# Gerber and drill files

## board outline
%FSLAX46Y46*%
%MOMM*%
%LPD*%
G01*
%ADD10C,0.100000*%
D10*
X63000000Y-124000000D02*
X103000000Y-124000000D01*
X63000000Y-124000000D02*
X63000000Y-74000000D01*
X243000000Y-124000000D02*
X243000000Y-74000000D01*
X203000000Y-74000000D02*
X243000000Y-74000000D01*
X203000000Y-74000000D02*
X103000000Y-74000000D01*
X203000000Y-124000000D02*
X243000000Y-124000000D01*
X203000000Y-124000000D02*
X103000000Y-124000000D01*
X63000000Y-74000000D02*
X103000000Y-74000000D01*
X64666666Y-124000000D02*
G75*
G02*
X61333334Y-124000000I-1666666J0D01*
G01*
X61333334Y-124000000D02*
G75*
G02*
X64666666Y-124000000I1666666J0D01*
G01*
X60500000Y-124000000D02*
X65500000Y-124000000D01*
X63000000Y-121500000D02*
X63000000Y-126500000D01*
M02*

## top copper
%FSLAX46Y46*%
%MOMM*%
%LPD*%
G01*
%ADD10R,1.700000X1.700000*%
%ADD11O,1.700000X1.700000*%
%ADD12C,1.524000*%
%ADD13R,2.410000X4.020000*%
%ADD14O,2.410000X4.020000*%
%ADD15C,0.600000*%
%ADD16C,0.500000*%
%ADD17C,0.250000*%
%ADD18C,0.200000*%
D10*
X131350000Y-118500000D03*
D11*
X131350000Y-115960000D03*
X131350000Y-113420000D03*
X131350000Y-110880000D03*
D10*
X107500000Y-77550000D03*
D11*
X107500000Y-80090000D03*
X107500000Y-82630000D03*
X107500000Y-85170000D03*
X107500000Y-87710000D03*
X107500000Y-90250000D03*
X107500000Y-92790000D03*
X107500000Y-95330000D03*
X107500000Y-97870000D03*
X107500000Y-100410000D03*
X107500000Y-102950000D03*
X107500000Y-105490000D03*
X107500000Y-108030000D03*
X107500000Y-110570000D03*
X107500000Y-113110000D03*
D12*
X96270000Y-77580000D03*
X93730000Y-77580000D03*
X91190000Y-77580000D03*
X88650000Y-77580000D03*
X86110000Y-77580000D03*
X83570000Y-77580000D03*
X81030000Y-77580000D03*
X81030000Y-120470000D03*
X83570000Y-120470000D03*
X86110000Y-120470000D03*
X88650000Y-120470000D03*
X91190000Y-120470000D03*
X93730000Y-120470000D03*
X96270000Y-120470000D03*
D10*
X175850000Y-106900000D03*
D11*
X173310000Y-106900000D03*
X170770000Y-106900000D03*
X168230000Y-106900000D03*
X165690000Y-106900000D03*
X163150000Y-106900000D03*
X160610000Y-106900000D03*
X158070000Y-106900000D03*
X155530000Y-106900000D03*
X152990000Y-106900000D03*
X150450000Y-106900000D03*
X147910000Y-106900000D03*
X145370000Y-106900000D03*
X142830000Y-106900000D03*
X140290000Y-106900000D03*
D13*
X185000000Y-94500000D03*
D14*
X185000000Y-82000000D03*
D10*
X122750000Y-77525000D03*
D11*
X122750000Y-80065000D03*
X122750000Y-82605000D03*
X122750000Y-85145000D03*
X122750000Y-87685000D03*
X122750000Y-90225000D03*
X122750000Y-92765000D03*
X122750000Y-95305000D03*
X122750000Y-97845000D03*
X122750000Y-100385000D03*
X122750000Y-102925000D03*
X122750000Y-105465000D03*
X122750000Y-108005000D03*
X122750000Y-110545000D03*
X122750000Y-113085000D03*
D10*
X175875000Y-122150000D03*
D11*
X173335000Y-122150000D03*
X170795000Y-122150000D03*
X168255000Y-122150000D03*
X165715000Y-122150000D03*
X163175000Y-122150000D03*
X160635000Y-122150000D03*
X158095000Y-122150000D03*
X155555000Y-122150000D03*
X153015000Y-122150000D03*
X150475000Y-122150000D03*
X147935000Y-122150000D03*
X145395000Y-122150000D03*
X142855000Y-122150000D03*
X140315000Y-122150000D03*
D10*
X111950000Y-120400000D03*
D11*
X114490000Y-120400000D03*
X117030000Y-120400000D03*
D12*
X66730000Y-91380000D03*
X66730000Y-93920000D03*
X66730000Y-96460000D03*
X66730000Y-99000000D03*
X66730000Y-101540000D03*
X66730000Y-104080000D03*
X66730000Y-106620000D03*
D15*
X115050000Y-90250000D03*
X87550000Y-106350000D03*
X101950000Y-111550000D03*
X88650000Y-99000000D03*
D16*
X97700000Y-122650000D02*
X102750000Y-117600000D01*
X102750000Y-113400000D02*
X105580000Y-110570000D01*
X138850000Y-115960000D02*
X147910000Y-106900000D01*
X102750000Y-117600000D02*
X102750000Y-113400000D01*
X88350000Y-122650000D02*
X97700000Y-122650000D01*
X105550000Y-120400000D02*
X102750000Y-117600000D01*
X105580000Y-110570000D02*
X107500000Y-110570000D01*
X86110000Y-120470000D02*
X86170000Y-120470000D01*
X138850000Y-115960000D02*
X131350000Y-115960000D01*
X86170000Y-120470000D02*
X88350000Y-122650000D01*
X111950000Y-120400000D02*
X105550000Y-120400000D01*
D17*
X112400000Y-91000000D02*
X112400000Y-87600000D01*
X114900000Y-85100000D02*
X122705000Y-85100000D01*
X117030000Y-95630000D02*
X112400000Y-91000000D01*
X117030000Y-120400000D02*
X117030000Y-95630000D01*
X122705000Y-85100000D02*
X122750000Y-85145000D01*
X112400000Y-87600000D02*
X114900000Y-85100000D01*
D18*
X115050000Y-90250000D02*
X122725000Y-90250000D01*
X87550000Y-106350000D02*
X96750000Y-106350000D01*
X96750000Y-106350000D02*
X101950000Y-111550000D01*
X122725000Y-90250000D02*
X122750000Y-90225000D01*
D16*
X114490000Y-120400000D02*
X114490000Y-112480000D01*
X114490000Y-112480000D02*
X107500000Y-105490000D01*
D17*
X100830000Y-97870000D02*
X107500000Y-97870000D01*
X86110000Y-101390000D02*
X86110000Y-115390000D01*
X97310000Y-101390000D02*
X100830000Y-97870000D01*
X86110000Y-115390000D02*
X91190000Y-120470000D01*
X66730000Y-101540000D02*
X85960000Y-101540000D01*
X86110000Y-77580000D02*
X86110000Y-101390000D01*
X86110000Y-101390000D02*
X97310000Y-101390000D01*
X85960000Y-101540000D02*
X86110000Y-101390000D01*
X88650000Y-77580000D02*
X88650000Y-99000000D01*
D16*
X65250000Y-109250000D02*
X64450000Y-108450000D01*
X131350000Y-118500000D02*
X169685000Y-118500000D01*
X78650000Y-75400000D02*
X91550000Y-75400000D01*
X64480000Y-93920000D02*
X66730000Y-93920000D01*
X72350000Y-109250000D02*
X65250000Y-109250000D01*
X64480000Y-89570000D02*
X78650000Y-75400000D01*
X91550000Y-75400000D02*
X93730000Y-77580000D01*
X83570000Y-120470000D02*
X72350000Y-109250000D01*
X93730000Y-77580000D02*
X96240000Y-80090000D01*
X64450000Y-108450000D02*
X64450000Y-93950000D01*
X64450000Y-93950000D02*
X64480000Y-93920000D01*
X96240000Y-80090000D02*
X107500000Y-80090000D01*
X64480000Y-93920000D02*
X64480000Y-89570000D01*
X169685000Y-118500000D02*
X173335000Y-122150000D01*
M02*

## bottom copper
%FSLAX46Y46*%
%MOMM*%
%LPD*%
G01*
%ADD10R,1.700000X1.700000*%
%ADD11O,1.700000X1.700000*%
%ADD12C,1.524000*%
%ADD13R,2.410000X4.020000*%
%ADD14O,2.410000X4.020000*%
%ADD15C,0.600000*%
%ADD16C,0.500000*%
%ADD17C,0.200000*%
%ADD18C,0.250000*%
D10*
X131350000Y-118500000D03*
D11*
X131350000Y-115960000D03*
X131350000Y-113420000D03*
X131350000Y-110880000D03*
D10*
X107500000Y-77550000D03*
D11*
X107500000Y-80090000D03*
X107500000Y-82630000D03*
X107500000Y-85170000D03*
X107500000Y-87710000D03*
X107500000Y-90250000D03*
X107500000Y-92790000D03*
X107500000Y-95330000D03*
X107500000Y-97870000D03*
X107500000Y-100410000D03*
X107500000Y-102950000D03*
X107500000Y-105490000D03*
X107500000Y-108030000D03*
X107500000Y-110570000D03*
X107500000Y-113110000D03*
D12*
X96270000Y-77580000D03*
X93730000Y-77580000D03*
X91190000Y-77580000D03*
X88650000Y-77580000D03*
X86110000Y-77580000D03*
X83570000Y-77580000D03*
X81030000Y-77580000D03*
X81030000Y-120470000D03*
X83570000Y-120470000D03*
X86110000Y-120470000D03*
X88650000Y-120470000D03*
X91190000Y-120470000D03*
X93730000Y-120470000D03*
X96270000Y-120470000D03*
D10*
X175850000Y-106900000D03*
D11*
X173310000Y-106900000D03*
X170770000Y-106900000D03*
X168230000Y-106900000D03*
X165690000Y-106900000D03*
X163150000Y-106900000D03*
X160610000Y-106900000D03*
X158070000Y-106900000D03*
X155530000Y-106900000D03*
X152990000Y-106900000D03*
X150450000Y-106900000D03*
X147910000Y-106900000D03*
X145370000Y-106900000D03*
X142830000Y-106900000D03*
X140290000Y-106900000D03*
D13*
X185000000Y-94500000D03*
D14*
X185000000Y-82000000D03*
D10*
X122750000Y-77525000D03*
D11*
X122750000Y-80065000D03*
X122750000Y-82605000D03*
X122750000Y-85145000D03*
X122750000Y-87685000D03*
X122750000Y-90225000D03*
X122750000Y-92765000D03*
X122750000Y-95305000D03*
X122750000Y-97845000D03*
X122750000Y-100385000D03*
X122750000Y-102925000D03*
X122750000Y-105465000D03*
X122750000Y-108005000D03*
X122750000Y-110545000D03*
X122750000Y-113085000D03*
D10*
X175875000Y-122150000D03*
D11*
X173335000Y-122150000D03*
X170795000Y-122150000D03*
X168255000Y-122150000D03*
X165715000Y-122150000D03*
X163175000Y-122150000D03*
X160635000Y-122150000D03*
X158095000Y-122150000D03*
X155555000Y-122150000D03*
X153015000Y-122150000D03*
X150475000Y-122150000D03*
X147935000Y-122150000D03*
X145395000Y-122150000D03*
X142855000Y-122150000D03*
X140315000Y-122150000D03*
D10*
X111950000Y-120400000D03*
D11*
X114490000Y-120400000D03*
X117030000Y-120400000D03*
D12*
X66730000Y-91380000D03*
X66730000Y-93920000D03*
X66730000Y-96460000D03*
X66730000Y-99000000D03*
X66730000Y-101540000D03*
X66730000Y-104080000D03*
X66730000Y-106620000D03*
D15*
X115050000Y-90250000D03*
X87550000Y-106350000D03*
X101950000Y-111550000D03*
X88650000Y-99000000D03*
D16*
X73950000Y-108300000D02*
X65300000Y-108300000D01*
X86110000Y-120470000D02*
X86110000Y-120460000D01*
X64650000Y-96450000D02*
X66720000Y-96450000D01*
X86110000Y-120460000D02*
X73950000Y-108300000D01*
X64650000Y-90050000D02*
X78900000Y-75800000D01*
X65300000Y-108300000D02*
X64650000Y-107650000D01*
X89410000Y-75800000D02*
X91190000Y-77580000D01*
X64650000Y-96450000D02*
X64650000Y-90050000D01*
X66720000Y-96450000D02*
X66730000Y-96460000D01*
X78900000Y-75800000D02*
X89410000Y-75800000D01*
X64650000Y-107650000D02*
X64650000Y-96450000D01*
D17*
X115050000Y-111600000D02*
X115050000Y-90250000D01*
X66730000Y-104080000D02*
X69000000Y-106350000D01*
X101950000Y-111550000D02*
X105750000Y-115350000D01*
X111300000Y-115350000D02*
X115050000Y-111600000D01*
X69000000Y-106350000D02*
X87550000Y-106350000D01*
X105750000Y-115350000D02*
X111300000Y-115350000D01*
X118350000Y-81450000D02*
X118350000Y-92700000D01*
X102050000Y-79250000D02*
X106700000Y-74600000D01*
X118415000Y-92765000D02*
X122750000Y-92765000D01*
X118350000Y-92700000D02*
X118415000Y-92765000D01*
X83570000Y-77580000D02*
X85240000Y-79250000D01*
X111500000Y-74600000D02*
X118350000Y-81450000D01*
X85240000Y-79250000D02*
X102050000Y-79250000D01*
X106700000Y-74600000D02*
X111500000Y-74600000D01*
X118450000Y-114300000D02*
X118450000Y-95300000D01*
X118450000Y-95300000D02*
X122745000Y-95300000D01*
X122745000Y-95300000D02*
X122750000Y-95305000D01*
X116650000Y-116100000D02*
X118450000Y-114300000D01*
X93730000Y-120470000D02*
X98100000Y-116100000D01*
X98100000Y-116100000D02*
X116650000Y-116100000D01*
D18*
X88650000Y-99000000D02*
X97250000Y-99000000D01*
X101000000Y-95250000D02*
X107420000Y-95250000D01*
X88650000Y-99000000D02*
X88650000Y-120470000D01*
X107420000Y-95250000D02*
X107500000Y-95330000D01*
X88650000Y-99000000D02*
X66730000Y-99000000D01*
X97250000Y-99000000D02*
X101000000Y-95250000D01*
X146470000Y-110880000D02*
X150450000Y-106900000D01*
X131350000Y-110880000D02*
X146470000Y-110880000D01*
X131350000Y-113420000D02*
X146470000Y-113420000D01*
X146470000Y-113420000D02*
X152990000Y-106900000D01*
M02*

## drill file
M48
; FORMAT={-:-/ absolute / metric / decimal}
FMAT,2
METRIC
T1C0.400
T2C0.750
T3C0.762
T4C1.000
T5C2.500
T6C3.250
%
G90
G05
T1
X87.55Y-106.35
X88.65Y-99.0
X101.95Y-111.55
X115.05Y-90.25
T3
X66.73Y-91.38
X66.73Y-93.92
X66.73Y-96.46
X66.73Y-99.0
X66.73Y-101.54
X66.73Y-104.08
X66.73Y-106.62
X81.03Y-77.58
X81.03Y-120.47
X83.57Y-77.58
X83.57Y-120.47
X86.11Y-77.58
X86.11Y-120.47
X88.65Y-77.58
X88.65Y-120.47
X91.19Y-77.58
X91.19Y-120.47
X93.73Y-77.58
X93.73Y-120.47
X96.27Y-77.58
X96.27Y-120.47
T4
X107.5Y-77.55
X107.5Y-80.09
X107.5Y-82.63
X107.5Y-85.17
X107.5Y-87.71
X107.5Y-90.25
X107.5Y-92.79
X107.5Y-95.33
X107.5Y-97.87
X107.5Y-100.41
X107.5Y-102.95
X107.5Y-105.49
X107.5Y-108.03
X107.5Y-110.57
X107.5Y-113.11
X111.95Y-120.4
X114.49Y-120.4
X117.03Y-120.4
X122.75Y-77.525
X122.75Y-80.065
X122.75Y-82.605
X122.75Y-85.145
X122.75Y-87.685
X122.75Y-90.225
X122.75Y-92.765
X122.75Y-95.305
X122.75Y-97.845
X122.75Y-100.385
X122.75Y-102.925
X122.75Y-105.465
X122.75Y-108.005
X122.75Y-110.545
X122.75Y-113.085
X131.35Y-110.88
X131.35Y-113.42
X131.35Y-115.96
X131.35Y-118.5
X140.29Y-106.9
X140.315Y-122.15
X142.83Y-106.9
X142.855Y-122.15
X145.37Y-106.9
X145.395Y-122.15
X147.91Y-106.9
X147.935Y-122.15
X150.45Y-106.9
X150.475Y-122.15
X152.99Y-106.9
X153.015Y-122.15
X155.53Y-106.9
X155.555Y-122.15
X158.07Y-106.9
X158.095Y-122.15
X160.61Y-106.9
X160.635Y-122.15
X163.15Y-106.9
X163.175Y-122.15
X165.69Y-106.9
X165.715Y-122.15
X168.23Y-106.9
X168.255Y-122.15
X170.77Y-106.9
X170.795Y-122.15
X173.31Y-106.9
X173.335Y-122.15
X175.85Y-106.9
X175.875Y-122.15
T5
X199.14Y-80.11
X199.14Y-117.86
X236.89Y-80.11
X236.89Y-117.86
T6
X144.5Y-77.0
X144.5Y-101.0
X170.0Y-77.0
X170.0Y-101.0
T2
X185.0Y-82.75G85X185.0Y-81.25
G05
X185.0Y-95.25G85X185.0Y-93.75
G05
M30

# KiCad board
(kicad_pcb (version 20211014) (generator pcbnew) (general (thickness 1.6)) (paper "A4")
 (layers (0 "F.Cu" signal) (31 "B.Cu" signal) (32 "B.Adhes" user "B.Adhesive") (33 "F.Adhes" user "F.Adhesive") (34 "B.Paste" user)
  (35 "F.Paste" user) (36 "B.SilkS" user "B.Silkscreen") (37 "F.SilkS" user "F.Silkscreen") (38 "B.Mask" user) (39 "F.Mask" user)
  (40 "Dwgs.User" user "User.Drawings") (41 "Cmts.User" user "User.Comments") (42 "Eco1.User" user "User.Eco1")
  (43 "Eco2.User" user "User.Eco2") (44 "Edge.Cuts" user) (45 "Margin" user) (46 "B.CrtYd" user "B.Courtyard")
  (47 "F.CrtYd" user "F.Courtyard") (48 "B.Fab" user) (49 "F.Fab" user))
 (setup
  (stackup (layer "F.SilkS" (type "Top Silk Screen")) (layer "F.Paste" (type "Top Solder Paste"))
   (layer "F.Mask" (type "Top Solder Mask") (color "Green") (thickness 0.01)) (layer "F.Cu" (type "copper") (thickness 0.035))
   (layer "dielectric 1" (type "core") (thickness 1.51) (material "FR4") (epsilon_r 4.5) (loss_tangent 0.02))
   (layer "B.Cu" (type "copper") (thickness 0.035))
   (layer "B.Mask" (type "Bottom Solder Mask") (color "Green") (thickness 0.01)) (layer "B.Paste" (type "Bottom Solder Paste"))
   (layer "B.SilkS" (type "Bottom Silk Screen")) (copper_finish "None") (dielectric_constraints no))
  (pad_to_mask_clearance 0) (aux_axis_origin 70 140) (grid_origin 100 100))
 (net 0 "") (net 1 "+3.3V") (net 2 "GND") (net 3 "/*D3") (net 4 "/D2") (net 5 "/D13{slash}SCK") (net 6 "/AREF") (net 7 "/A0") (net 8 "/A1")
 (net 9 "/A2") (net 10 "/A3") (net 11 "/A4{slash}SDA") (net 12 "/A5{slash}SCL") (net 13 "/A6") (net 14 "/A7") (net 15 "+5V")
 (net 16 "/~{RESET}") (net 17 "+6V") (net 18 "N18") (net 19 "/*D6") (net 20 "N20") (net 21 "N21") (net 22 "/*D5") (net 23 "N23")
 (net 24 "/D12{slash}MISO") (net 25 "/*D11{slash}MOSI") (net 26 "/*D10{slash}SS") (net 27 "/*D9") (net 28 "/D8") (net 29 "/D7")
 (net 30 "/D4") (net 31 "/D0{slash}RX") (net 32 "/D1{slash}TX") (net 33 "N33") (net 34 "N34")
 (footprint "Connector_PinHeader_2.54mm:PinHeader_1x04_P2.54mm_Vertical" (layer "F.Cu") (at 131.35 118.5 180)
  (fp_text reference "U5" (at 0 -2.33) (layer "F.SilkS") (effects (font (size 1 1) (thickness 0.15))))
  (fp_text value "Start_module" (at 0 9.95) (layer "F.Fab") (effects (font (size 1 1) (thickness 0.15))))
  (pad "1" thru_hole rect (at 0 0 180) (size 1.7 1.7) (drill 1) (layers *.Cu *.Mask) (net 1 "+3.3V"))
  (pad "2" thru_hole oval (at 0 2.54 180) (size 1.7 1.7) (drill 1) (layers *.Cu *.Mask) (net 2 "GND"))
  (pad "3" thru_hole oval (at 0 5.08 180) (size 1.7 1.7) (drill 1) (layers *.Cu *.Mask) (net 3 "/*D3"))
  (pad "4" thru_hole oval (at 0 7.62 180) (size 1.7 1.7) (drill 1) (layers *.Cu *.Mask) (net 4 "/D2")))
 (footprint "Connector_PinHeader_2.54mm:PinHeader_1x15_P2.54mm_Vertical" (layer "F.Cu") (at 107.5 77.55)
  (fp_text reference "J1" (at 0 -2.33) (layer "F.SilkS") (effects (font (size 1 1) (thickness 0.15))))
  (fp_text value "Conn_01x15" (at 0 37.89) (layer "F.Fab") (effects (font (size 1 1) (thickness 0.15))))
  (pad "1" thru_hole rect (at 0 0) (size 1.7 1.7) (drill 1) (layers *.Cu *.Mask) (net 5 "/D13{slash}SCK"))
  (pad "2" thru_hole oval (at 0 2.54) (size 1.7 1.7) (drill 1) (layers *.Cu *.Mask) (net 1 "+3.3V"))
  (pad "3" thru_hole oval (at 0 5.08) (size 1.7 1.7) (drill 1) (layers *.Cu *.Mask) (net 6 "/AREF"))
  (pad "4" thru_hole oval (at 0 7.62) (size 1.7 1.7) (drill 1) (layers *.Cu *.Mask) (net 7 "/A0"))
  (pad "5" thru_hole oval (at 0 10.16) (size 1.7 1.7) (drill 1) (layers *.Cu *.Mask) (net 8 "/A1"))
  (pad "6" thru_hole oval (at 0 12.7) (size 1.7 1.7) (drill 1) (layers *.Cu *.Mask) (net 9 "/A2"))
  (pad "7" thru_hole oval (at 0 15.24) (size 1.7 1.7) (drill 1) (layers *.Cu *.Mask) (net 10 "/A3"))
  (pad "8" thru_hole oval (at 0 17.78) (size 1.7 1.7) (drill 1) (layers *.Cu *.Mask) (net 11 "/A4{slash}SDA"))
  (pad "9" thru_hole oval (at 0 20.32) (size 1.7 1.7) (drill 1) (layers *.Cu *.Mask) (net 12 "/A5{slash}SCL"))
  (pad "10" thru_hole oval (at 0 22.86) (size 1.7 1.7) (drill 1) (layers *.Cu *.Mask) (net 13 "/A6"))
  (pad "11" thru_hole oval (at 0 25.4) (size 1.7 1.7) (drill 1) (layers *.Cu *.Mask) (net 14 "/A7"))
  (pad "12" thru_hole oval (at 0 27.94) (size 1.7 1.7) (drill 1) (layers *.Cu *.Mask) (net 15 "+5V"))
  (pad "13" thru_hole oval (at 0 30.48) (size 1.7 1.7) (drill 1) (layers *.Cu *.Mask) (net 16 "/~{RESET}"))
  (pad "14" thru_hole oval (at 0 33.02) (size 1.7 1.7) (drill 1) (layers *.Cu *.Mask) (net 2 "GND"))
  (pad "15" thru_hole oval (at 0 35.56) (size 1.7 1.7) (drill 1) (layers *.Cu *.Mask) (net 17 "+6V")))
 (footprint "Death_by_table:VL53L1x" (layer "F.Cu") (at 96.27 77.58 180)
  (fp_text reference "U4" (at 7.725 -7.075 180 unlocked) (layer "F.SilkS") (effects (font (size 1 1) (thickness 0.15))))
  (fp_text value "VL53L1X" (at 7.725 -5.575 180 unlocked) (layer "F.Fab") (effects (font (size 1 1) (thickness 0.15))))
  (pad "1" thru_hole circle (at 0 0 180) (size 1.524 1.524) (drill 0.762) (layers *.Cu *.Mask) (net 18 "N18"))
  (pad "2" thru_hole circle (at 2.54 0 180) (size 1.524 1.524) (drill 0.762) (layers *.Cu *.Mask) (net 1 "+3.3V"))
  (pad "3" thru_hole circle (at 5.08 0 180) (size 1.524 1.524) (drill 0.762) (layers *.Cu *.Mask) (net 2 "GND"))
  (pad "4" thru_hole circle (at 7.62 0 180) (size 1.524 1.524) (drill 0.762) (layers *.Cu *.Mask) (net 11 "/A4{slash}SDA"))
  (pad "5" thru_hole circle (at 10.16 0 180) (size 1.524 1.524) (drill 0.762) (layers *.Cu *.Mask) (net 12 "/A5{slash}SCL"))
  (pad "6" thru_hole circle (at 12.7 0 180) (size 1.524 1.524) (drill 0.762) (layers *.Cu *.Mask) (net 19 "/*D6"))
  (pad "7" thru_hole circle (at 15.24 0 180) (size 1.524 1.524) (drill 0.762) (layers *.Cu *.Mask) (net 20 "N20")))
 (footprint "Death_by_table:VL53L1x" (layer "F.Cu") (at 81.03 120.47)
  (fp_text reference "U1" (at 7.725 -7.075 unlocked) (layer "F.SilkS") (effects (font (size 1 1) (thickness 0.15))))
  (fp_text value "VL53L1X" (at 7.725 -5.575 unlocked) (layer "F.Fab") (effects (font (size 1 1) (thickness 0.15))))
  (pad "1" thru_hole circle (at 0 0) (size 1.524 1.524) (drill 0.762) (layers *.Cu *.Mask) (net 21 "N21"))
  (pad "2" thru_hole circle (at 2.54 0) (size 1.524 1.524) (drill 0.762) (layers *.Cu *.Mask) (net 1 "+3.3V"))
  (pad "3" thru_hole circle (at 5.08 0) (size 1.524 1.524) (drill 0.762) (layers *.Cu *.Mask) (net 2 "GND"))
  (pad "4" thru_hole circle (at 7.62 0) (size 1.524 1.524) (drill 0.762) (layers *.Cu *.Mask) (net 11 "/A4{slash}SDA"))
  (pad "5" thru_hole circle (at 10.16 0) (size 1.524 1.524) (drill 0.762) (layers *.Cu *.Mask) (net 12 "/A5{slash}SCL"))
  (pad "6" thru_hole circle (at 12.7 0) (size 1.524 1.524) (drill 0.762) (layers *.Cu *.Mask) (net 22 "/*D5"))
  (pad "7" thru_hole circle (at 15.24 0) (size 1.524 1.524) (drill 0.762) (layers *.Cu *.Mask) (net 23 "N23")))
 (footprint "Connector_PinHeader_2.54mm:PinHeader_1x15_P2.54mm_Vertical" (layer "F.Cu") (at 175.85 106.9 -90)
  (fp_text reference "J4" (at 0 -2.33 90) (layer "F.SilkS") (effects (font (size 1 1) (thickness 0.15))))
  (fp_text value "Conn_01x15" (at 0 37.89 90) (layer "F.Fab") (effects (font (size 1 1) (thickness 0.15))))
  (pad "1" thru_hole rect (at 0 0 270) (size 1.7 1.7) (drill 1) (layers *.Cu *.Mask) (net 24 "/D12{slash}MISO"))
  (pad "2" thru_hole oval (at 0 2.54 270) (size 1.7 1.7) (drill 1) (layers *.Cu *.Mask) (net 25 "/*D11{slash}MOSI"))
  (pad "3" thru_hole oval (at 0 5.08 270) (size 1.7 1.7) (drill 1) (layers *.Cu *.Mask) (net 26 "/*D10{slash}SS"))
  (pad "4" thru_hole oval (at 0 7.62 270) (size 1.7 1.7) (drill 1) (layers *.Cu *.Mask) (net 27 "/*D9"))
  (pad "5" thru_hole oval (at 0 10.16 270) (size 1.7 1.7) (drill 1) (layers *.Cu *.Mask) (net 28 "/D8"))
  (pad "6" thru_hole oval (at 0 12.7 270) (size 1.7 1.7) (drill 1) (layers *.Cu *.Mask) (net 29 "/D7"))
  (pad "7" thru_hole oval (at 0 15.24 270) (size 1.7 1.7) (drill 1) (layers *.Cu *.Mask) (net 19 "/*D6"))
  (pad "8" thru_hole oval (at 0 17.78 270) (size 1.7 1.7) (drill 1) (layers *.Cu *.Mask) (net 22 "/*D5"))
  (pad "9" thru_hole oval (at 0 20.32 270) (size 1.7 1.7) (drill 1) (layers *.Cu *.Mask) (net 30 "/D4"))
  (pad "10" thru_hole oval (at 0 22.86 270) (size 1.7 1.7) (drill 1) (layers *.Cu *.Mask) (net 3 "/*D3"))
  (pad "11" thru_hole oval (at 0 25.4 270) (size 1.7 1.7) (drill 1) (layers *.Cu *.Mask) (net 4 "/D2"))
  (pad "12" thru_hole oval (at 0 27.94 270) (size 1.7 1.7) (drill 1) (layers *.Cu *.Mask) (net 2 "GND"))
  (pad "13" thru_hole oval (at 0 30.48 270) (size 1.7 1.7) (drill 1) (layers *.Cu *.Mask) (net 16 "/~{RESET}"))
  (pad "14" thru_hole oval (at 0 33.02 270) (size 1.7 1.7) (drill 1) (layers *.Cu *.Mask) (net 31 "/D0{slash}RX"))
  (pad "15" thru_hole oval (at 0 35.56 270) (size 1.7 1.7) (drill 1) (layers *.Cu *.Mask) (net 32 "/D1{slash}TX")))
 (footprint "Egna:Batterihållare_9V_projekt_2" (layer "F.Cu") (at 185 74 180)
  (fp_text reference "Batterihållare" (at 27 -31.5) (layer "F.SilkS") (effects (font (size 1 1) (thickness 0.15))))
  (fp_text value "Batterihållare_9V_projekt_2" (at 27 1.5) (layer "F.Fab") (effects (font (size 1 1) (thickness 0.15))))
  (pad "" np_thru_hole circle (at 15 -27 180) (size 2.3 2.3) (drill 3.25) (layers F&B.Cu *.Mask))
  (pad "" np_thru_hole circle (at 40.5 -3 180) (size 2.3 2.3) (drill 3.25) (layers F&B.Cu *.Mask))
  (pad "" np_thru_hole circle (at 15 -3 180) (size 2.3 2.3) (drill 3.25) (layers F&B.Cu *.Mask))
  (pad "" np_thru_hole circle (at 40.5 -27 180) (size 2.3 2.3) (drill 3.25) (layers F&B.Cu *.Mask))
  (pad "1" thru_hole rect (at 0 -20.5 180) (size 2.41 4.02) (drill oval 0.75 2.25) (layers *.Cu *.Mask))
  (pad "2" thru_hole oval (at 0 -8 180) (size 2.41 4.02) (drill oval 0.75 2.25) (layers *.Cu *.Mask)))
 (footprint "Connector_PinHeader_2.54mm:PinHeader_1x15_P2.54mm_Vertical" (layer "F.Cu") (at 122.75 77.525)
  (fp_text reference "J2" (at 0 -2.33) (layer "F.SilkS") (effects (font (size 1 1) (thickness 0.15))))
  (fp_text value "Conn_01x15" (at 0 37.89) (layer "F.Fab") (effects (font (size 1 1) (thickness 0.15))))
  (pad "1" thru_hole rect (at 0 0) (size 1.7 1.7) (drill 1) (layers *.Cu *.Mask) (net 24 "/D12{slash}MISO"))
  (pad "2" thru_hole oval (at 0 2.54) (size 1.7 1.7) (drill 1) (layers *.Cu *.Mask) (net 25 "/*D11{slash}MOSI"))
  (pad "3" thru_hole oval (at 0 5.08) (size 1.7 1.7) (drill 1) (layers *.Cu *.Mask) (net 26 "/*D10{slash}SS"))
  (pad "4" thru_hole oval (at 0 7.62) (size 1.7 1.7) (drill 1) (layers *.Cu *.Mask) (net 27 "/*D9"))
  (pad "5" thru_hole oval (at 0 10.16) (size 1.7 1.7) (drill 1) (layers *.Cu *.Mask) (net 28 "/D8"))
  (pad "6" thru_hole oval (at 0 12.7) (size 1.7 1.7) (drill 1) (layers *.Cu *.Mask) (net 29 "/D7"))
  (pad "7" thru_hole oval (at 0 15.24) (size 1.7 1.7) (drill 1) (layers *.Cu *.Mask) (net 19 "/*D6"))
  (pad "8" thru_hole oval (at 0 17.78) (size 1.7 1.7) (drill 1) (layers *.Cu *.Mask) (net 22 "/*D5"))
  (pad "9" thru_hole oval (at 0 20.32) (size 1.7 1.7) (drill 1) (layers *.Cu *.Mask) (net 30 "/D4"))
  (pad "10" thru_hole oval (at 0 22.86) (size 1.7 1.7) (drill 1) (layers *.Cu *.Mask) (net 3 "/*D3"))
  (pad "11" thru_hole oval (at 0 25.4) (size 1.7 1.7) (drill 1) (layers *.Cu *.Mask) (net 4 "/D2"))
  (pad "12" thru_hole oval (at 0 27.94) (size 1.7 1.7) (drill 1) (layers *.Cu *.Mask) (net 2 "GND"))
  (pad "13" thru_hole oval (at 0 30.48) (size 1.7 1.7) (drill 1) (layers *.Cu *.Mask) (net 16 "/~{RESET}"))
  (pad "14" thru_hole oval (at 0 33.02) (size 1.7 1.7) (drill 1) (layers *.Cu *.Mask) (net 31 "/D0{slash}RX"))
  (pad "15" thru_hole oval (at 0 35.56) (size 1.7 1.7) (drill 1) (layers *.Cu *.Mask) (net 32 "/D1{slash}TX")))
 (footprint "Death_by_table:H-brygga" (layer "F.Cu") (at 195.14 121.86)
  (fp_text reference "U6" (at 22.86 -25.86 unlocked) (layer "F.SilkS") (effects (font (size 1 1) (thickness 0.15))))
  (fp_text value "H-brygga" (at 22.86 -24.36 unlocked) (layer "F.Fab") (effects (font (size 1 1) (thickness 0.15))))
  (pad "" np_thru_hole circle (at 4 -4) (size 2.5 2.5) (drill 2.5) (layers F&B.Cu *.Mask))
  (pad "" np_thru_hole circle (at 41.75 -41.75) (size 2.5 2.5) (drill 2.5) (layers F&B.Cu *.Mask))
  (pad "" np_thru_hole circle (at 4 -41.75) (size 2.5 2.5) (drill 2.5) (layers F&B.Cu *.Mask))
  (pad "" np_thru_hole circle (at 41.75 -4) (size 2.5 2.5) (drill 2.5) (layers F&B.Cu *.Mask)))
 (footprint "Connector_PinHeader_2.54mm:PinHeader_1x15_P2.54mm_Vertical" (layer "F.Cu") (at 175.875 122.15 -90)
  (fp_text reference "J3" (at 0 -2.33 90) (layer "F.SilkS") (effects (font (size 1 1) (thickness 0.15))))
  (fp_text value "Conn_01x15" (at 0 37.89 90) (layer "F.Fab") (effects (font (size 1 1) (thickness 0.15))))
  (pad "1" thru_hole rect (at 0 0 270) (size 1.7 1.7) (drill 1) (layers *.Cu *.Mask) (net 5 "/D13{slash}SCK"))
  (pad "2" thru_hole oval (at 0 2.54 270) (size 1.7 1.7) (drill 1) (layers *.Cu *.Mask) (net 1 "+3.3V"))
  (pad "3" thru_hole oval (at 0 5.08 270) (size 1.7 1.7) (drill 1) (layers *.Cu *.Mask) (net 6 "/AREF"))
  (pad "4" thru_hole oval (at 0 7.62 270) (size 1.7 1.7) (drill 1) (layers *.Cu *.Mask) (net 7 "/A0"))
  (pad "5" thru_hole oval (at 0 10.16 270) (size 1.7 1.7) (drill 1) (layers *.Cu *.Mask) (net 8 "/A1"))
  (pad "6" thru_hole oval (at 0 12.7 270) (size 1.7 1.7) (drill 1) (layers *.Cu *.Mask) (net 9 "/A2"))
  (pad "7" thru_hole oval (at 0 15.24 270) (size 1.7 1.7) (drill 1) (layers *.Cu *.Mask) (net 10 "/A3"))
  (pad "8" thru_hole oval (at 0 17.78 270) (size 1.7 1.7) (drill 1) (layers *.Cu *.Mask) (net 11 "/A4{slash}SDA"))
  (pad "9" thru_hole oval (at 0 20.32 270) (size 1.7 1.7) (drill 1) (layers *.Cu *.Mask) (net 12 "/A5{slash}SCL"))
  (pad "10" thru_hole oval (at 0 22.86 270) (size 1.7 1.7) (drill 1) (layers *.Cu *.Mask) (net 13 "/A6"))
  (pad "11" thru_hole oval (at 0 25.4 270) (size 1.7 1.7) (drill 1) (layers *.Cu *.Mask) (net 14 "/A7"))
  (pad "12" thru_hole oval (at 0 27.94 270) (size 1.7 1.7) (drill 1) (layers *.Cu *.Mask) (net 15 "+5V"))
  (pad "13" thru_hole oval (at 0 30.48 270) (size 1.7 1.7) (drill 1) (layers *.Cu *.Mask) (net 16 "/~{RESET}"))
  (pad "14" thru_hole oval (at 0 33.02 270) (size 1.7 1.7) (drill 1) (layers *.Cu *.Mask) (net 2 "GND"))
  (pad "15" thru_hole oval (at 0 35.56 270) (size 1.7 1.7) (drill 1) (layers *.Cu *.Mask) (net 17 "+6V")))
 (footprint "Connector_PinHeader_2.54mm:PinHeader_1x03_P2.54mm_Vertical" (layer "F.Cu") (at 111.95 120.4 90)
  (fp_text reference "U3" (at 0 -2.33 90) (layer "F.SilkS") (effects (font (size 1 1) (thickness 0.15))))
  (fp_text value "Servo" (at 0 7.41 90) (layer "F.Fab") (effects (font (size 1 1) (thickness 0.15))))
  (pad "1" thru_hole rect (at 0 0 90) (size 1.7 1.7) (drill 1) (layers *.Cu *.Mask) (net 2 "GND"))
  (pad "2" thru_hole oval (at 0 2.54 90) (size 1.7 1.7) (drill 1) (layers *.Cu *.Mask) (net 15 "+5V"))
  (pad "3" thru_hole oval (at 0 5.08 90) (size 1.7 1.7) (drill 1) (layers *.Cu *.Mask) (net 27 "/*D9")))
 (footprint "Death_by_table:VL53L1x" (layer "F.Cu") (at 66.73 91.38 -90)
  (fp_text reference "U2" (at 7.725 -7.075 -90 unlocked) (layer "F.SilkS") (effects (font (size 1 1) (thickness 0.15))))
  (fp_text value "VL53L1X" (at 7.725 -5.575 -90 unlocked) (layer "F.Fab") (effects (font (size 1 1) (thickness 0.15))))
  (pad "1" thru_hole circle (at 0 0 270) (size 1.524 1.524) (drill 0.762) (layers *.Cu *.Mask) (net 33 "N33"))
  (pad "2" thru_hole circle (at 2.54 0 270) (size 1.524 1.524) (drill 0.762) (layers *.Cu *.Mask) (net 1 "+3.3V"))
  (pad "3" thru_hole circle (at 5.08 0 270) (size 1.524 1.524) (drill 0.762) (layers *.Cu *.Mask) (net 2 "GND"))
  (pad "4" thru_hole circle (at 7.62 0 270) (size 1.524 1.524) (drill 0.762) (layers *.Cu *.Mask) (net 11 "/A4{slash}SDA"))
  (pad "5" thru_hole circle (at 10.16 0 270) (size 1.524 1.524) (drill 0.762) (layers *.Cu *.Mask) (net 12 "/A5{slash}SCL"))
  (pad "6" thru_hole circle (at 12.7 0 270) (size 1.524 1.524) (drill 0.762) (layers *.Cu *.Mask) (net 29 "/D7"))
  (pad "7" thru_hole circle (at 15.24 0 270) (size 1.524 1.524) (drill 0.762) (layers *.Cu *.Mask) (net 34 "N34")))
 (gr_line (start 63 124) (end 103 124) (layer "Edge.Cuts") (width 0.1))
 (gr_line (start 63 124) (end 63 74) (layer "Edge.Cuts") (width 0.1))
 (gr_line (start 243 124) (end 243 74) (layer "Edge.Cuts") (width 0.1))
 (gr_line (start 203 74) (end 243 74) (layer "Edge.Cuts") (width 0.1))
 (gr_line (start 203 74) (end 103 74) (layer "Edge.Cuts") (width 0.1))
 (gr_line (start 203 124) (end 243 124) (layer "Edge.Cuts") (width 0.1))
 (gr_line (start 203 124) (end 103 124) (layer "Edge.Cuts") (width 0.1))
 (gr_line (start 63 74) (end 103 74) (layer "Edge.Cuts") (width 0.1))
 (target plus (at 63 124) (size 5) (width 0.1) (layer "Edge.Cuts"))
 (segment (start 97.7 122.65) (end 102.75 117.6) (width 0.5) (layer "F.Cu") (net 2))
 (segment (start 102.75 113.4) (end 105.58 110.57) (width 0.5) (layer "F.Cu") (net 2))
 (segment (start 138.85 115.96) (end 147.91 106.9) (width 0.5) (layer "F.Cu") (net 2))
 (segment (start 102.75 117.6) (end 102.75 113.4) (width 0.5) (layer "F.Cu") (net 2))
 (segment (start 88.35 122.65) (end 97.7 122.65) (width 0.5) (layer "F.Cu") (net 2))
 (segment (start 105.55 120.4) (end 102.75 117.6) (width 0.5) (layer "F.Cu") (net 2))
 (segment (start 105.58 110.57) (end 107.5 110.57) (width 0.5) (layer "F.Cu") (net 2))
 (segment (start 86.11 120.47) (end 86.17 120.47) (width 0.5) (layer "F.Cu") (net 2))
 (segment (start 138.85 115.96) (end 131.35 115.96) (width 0.5) (layer "F.Cu") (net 2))
 (segment (start 86.17 120.47) (end 88.35 122.65) (width 0.5) (layer "F.Cu") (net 2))
 (segment (start 111.95 120.4) (end 105.55 120.4) (width 0.5) (layer "F.Cu") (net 2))
 (segment (start 73.95 108.3) (end 65.3 108.3) (width 0.5) (layer "B.Cu") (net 2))
 (segment (start 86.11 120.47) (end 86.11 120.46) (width 0.5) (layer "B.Cu") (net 2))
 (segment (start 64.65 96.45) (end 66.72 96.45) (width 0.5) (layer "B.Cu") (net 2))
 (segment (start 86.11 120.46) (end 73.95 108.3) (width 0.5) (layer "B.Cu") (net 2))
 (segment (start 64.65 90.05) (end 78.9 75.8) (width 0.5) (layer "B.Cu") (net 2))
 (segment (start 65.3 108.3) (end 64.65 107.65) (width 0.5) (layer "B.Cu") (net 2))
 (segment (start 89.41 75.8) (end 91.19 77.58) (width 0.5) (layer "B.Cu") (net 2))
 (segment (start 64.65 96.45) (end 64.65 90.05) (width 0.5) (layer "B.Cu") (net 2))
 (segment (start 66.72 96.45) (end 66.73 96.46) (width 0.5) (layer "B.Cu") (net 2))
 (segment (start 78.9 75.8) (end 89.41 75.8) (width 0.5) (layer "B.Cu") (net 2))
 (segment (start 64.65 107.65) (end 64.65 96.45) (width 0.5) (layer "B.Cu") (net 2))
 (segment (start 112.4 91) (end 112.4 87.6) (width 0.25) (layer "F.Cu") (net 27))
 (segment (start 114.9 85.1) (end 122.705 85.1) (width 0.25) (layer "F.Cu") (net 27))
 (segment (start 117.03 95.63) (end 112.4 91) (width 0.25) (layer "F.Cu") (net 27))
 (segment (start 117.03 120.4) (end 117.03 95.63) (width 0.25) (layer "F.Cu") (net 27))
 (segment (start 122.705 85.1) (end 122.75 85.145) (width 0.25) (layer "F.Cu") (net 27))
 (segment (start 112.4 87.6) (end 114.9 85.1) (width 0.25) (layer "F.Cu") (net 27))
 (segment (start 115.05 90.25) (end 122.725 90.25) (width 0.2) (layer "F.Cu") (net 29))
 (segment (start 87.55 106.35) (end 96.75 106.35) (width 0.2) (layer "F.Cu") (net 29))
 (segment (start 96.75 106.35) (end 101.95 111.55) (width 0.2) (layer "F.Cu") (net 29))
 (segment (start 122.725 90.25) (end 122.75 90.225) (width 0.2) (layer "F.Cu") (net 29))
 (via (at 115.05 90.25) (size 0.6) (drill 0.4) (layers "F.Cu" "B.Cu") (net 29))
 (via (at 87.55 106.35) (size 0.6) (drill 0.4) (layers "F.Cu" "B.Cu") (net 29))
 (via (at 101.95 111.55) (size 0.6) (drill 0.4) (layers "F.Cu" "B.Cu") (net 29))
 (segment (start 115.05 111.6) (end 115.05 90.25) (width 0.2) (layer "B.Cu") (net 29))
 (segment (start 66.73 104.08) (end 69 106.35) (width 0.2) (layer "B.Cu") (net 29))
 (segment (start 101.95 111.55) (end 105.75 115.35) (width 0.2) (layer "B.Cu") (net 29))
 (segment (start 111.3 115.35) (end 115.05 111.6) (width 0.2) (layer "B.Cu") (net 29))
 (segment (start 69 106.35) (end 87.55 106.35) (width 0.2) (layer "B.Cu") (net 29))
 (segment (start 105.75 115.35) (end 111.3 115.35) (width 0.2) (layer "B.Cu") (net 29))
 (segment (start 118.35 81.45) (end 118.35 92.7) (width 0.2) (layer "B.Cu") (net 19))
 (segment (start 102.05 79.25) (end 106.7 74.6) (width 0.2) (layer "B.Cu") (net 19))
 (segment (start 118.415 92.765) (end 122.75 92.765) (width 0.2) (layer "B.Cu") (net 19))
 (segment (start 118.35 92.7) (end 118.415 92.765) (width 0.2) (layer "B.Cu") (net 19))
 (segment (start 83.57 77.58) (end 85.24 79.25) (width 0.2) (layer "B.Cu") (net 19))
 (segment (start 111.5 74.6) (end 118.35 81.45) (width 0.2) (layer "B.Cu") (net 19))
 (segment (start 85.24 79.25) (end 102.05 79.25) (width 0.2) (layer "B.Cu") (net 19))
 (segment (start 106.7 74.6) (end 111.5 74.6) (width 0.2) (layer "B.Cu") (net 19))
 (segment (start 118.45 114.3) (end 118.45 95.3) (width 0.2) (layer "B.Cu") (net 22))
 (segment (start 118.45 95.3) (end 122.745 95.3) (width 0.2) (layer "B.Cu") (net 22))
 (segment (start 122.745 95.3) (end 122.75 95.305) (width 0.2) (layer "B.Cu") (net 22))
 (segment (start 116.65 116.1) (end 118.45 114.3) (width 0.2) (layer "B.Cu") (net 22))
 (segment (start 93.73 120.47) (end 98.1 116.1) (width 0.2) (layer "B.Cu") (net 22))
 (segment (start 98.1 116.1) (end 116.65 116.1) (width 0.2) (layer "B.Cu") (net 22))
 (segment (start 114.49 120.4) (end 114.49 112.48) (width 0.5) (layer "F.Cu") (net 15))
 (segment (start 114.49 112.48) (end 107.5 105.49) (width 0.5) (layer "F.Cu") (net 15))
 (segment (start 100.83 97.87) (end 107.5 97.87) (width 0.25) (layer "F.Cu") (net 12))
 (segment (start 86.11 101.39) (end 86.11 115.39) (width 0.25) (layer "F.Cu") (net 12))
 (segment (start 97.31 101.39) (end 100.83 97.87) (width 0.25) (layer "F.Cu") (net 12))
 (segment (start 86.11 115.39) (end 91.19 120.47) (width 0.25) (layer "F.Cu") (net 12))
 (segment (start 66.73 101.54) (end 85.96 101.54) (width 0.25) (layer "F.Cu") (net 12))
 (segment (start 86.11 77.58) (end 86.11 101.39) (width 0.25) (layer "F.Cu") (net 12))
 (segment (start 86.11 101.39) (end 97.31 101.39) (width 0.25) (layer "F.Cu") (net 12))
 (segment (start 85.96 101.54) (end 86.11 101.39) (width 0.25) (layer "F.Cu") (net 12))
 (segment (start 88.65 77.58) (end 88.65 99) (width 0.25) (layer "F.Cu") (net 11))
 (via (at 88.65 99) (size 0.6) (drill 0.4) (layers "F.Cu" "B.Cu") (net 11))
 (segment (start 88.65 99) (end 97.25 99) (width 0.25) (layer "B.Cu") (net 11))
 (segment (start 101 95.25) (end 107.42 95.25) (width 0.25) (layer "B.Cu") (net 11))
 (segment (start 88.65 99) (end 88.65 120.47) (width 0.25) (layer "B.Cu") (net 11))
 (segment (start 107.42 95.25) (end 107.5 95.33) (width 0.25) (layer "B.Cu") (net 11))
 (segment (start 88.65 99) (end 66.73 99) (width 0.25) (layer "B.Cu") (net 11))
 (segment (start 97.25 99) (end 101 95.25) (width 0.25) (layer "B.Cu") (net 11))
 (segment (start 146.47 110.88) (end 150.45 106.9) (width 0.25) (layer "B.Cu") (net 4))
 (segment (start 131.35 110.88) (end 146.47 110.88) (width 0.25) (layer "B.Cu") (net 4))
 (segment (start 131.35 113.42) (end 146.47 113.42) (width 0.25) (layer "B.Cu") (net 3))
 (segment (start 146.47 113.42) (end 152.99 106.9) (width 0.25) (layer "B.Cu") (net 3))
 (segment (start 65.25 109.25) (end 64.45 108.45) (width 0.5) (layer "F.Cu") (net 1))
 (segment (start 131.35 118.5) (end 169.685 118.5) (width 0.5) (layer "F.Cu") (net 1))
 (segment (start 78.65 75.4) (end 91.55 75.4) (width 0.5) (layer "F.Cu") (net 1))
 (segment (start 64.48 93.92) (end 66.73 93.92) (width 0.5) (layer "F.Cu") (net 1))
 (segment (start 72.35 109.25) (end 65.25 109.25) (width 0.5) (layer "F.Cu") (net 1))
 (segment (start 64.48 89.57) (end 78.65 75.4) (width 0.5) (layer "F.Cu") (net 1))
 (segment (start 91.55 75.4) (end 93.73 77.58) (width 0.5) (layer "F.Cu") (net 1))
 (segment (start 83.57 120.47) (end 72.35 109.25) (width 0.5) (layer "F.Cu") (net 1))
 (segment (start 93.73 77.58) (end 96.24 80.09) (width 0.5) (layer "F.Cu") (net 1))
 (segment (start 64.45 108.45) (end 64.45 93.95) (width 0.5) (layer "F.Cu") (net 1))
 (segment (start 64.45 93.95) (end 64.48 93.92) (width 0.5) (layer "F.Cu") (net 1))
 (segment (start 96.24 80.09) (end 107.5 80.09) (width 0.5) (layer "F.Cu") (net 1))
 (segment (start 64.48 93.92) (end 64.48 89.57) (width 0.5) (layer "F.Cu") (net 1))
 (segment (start 169.685 118.5) (end 173.335 122.15) (width 0.5) (layer "F.Cu") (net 1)))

